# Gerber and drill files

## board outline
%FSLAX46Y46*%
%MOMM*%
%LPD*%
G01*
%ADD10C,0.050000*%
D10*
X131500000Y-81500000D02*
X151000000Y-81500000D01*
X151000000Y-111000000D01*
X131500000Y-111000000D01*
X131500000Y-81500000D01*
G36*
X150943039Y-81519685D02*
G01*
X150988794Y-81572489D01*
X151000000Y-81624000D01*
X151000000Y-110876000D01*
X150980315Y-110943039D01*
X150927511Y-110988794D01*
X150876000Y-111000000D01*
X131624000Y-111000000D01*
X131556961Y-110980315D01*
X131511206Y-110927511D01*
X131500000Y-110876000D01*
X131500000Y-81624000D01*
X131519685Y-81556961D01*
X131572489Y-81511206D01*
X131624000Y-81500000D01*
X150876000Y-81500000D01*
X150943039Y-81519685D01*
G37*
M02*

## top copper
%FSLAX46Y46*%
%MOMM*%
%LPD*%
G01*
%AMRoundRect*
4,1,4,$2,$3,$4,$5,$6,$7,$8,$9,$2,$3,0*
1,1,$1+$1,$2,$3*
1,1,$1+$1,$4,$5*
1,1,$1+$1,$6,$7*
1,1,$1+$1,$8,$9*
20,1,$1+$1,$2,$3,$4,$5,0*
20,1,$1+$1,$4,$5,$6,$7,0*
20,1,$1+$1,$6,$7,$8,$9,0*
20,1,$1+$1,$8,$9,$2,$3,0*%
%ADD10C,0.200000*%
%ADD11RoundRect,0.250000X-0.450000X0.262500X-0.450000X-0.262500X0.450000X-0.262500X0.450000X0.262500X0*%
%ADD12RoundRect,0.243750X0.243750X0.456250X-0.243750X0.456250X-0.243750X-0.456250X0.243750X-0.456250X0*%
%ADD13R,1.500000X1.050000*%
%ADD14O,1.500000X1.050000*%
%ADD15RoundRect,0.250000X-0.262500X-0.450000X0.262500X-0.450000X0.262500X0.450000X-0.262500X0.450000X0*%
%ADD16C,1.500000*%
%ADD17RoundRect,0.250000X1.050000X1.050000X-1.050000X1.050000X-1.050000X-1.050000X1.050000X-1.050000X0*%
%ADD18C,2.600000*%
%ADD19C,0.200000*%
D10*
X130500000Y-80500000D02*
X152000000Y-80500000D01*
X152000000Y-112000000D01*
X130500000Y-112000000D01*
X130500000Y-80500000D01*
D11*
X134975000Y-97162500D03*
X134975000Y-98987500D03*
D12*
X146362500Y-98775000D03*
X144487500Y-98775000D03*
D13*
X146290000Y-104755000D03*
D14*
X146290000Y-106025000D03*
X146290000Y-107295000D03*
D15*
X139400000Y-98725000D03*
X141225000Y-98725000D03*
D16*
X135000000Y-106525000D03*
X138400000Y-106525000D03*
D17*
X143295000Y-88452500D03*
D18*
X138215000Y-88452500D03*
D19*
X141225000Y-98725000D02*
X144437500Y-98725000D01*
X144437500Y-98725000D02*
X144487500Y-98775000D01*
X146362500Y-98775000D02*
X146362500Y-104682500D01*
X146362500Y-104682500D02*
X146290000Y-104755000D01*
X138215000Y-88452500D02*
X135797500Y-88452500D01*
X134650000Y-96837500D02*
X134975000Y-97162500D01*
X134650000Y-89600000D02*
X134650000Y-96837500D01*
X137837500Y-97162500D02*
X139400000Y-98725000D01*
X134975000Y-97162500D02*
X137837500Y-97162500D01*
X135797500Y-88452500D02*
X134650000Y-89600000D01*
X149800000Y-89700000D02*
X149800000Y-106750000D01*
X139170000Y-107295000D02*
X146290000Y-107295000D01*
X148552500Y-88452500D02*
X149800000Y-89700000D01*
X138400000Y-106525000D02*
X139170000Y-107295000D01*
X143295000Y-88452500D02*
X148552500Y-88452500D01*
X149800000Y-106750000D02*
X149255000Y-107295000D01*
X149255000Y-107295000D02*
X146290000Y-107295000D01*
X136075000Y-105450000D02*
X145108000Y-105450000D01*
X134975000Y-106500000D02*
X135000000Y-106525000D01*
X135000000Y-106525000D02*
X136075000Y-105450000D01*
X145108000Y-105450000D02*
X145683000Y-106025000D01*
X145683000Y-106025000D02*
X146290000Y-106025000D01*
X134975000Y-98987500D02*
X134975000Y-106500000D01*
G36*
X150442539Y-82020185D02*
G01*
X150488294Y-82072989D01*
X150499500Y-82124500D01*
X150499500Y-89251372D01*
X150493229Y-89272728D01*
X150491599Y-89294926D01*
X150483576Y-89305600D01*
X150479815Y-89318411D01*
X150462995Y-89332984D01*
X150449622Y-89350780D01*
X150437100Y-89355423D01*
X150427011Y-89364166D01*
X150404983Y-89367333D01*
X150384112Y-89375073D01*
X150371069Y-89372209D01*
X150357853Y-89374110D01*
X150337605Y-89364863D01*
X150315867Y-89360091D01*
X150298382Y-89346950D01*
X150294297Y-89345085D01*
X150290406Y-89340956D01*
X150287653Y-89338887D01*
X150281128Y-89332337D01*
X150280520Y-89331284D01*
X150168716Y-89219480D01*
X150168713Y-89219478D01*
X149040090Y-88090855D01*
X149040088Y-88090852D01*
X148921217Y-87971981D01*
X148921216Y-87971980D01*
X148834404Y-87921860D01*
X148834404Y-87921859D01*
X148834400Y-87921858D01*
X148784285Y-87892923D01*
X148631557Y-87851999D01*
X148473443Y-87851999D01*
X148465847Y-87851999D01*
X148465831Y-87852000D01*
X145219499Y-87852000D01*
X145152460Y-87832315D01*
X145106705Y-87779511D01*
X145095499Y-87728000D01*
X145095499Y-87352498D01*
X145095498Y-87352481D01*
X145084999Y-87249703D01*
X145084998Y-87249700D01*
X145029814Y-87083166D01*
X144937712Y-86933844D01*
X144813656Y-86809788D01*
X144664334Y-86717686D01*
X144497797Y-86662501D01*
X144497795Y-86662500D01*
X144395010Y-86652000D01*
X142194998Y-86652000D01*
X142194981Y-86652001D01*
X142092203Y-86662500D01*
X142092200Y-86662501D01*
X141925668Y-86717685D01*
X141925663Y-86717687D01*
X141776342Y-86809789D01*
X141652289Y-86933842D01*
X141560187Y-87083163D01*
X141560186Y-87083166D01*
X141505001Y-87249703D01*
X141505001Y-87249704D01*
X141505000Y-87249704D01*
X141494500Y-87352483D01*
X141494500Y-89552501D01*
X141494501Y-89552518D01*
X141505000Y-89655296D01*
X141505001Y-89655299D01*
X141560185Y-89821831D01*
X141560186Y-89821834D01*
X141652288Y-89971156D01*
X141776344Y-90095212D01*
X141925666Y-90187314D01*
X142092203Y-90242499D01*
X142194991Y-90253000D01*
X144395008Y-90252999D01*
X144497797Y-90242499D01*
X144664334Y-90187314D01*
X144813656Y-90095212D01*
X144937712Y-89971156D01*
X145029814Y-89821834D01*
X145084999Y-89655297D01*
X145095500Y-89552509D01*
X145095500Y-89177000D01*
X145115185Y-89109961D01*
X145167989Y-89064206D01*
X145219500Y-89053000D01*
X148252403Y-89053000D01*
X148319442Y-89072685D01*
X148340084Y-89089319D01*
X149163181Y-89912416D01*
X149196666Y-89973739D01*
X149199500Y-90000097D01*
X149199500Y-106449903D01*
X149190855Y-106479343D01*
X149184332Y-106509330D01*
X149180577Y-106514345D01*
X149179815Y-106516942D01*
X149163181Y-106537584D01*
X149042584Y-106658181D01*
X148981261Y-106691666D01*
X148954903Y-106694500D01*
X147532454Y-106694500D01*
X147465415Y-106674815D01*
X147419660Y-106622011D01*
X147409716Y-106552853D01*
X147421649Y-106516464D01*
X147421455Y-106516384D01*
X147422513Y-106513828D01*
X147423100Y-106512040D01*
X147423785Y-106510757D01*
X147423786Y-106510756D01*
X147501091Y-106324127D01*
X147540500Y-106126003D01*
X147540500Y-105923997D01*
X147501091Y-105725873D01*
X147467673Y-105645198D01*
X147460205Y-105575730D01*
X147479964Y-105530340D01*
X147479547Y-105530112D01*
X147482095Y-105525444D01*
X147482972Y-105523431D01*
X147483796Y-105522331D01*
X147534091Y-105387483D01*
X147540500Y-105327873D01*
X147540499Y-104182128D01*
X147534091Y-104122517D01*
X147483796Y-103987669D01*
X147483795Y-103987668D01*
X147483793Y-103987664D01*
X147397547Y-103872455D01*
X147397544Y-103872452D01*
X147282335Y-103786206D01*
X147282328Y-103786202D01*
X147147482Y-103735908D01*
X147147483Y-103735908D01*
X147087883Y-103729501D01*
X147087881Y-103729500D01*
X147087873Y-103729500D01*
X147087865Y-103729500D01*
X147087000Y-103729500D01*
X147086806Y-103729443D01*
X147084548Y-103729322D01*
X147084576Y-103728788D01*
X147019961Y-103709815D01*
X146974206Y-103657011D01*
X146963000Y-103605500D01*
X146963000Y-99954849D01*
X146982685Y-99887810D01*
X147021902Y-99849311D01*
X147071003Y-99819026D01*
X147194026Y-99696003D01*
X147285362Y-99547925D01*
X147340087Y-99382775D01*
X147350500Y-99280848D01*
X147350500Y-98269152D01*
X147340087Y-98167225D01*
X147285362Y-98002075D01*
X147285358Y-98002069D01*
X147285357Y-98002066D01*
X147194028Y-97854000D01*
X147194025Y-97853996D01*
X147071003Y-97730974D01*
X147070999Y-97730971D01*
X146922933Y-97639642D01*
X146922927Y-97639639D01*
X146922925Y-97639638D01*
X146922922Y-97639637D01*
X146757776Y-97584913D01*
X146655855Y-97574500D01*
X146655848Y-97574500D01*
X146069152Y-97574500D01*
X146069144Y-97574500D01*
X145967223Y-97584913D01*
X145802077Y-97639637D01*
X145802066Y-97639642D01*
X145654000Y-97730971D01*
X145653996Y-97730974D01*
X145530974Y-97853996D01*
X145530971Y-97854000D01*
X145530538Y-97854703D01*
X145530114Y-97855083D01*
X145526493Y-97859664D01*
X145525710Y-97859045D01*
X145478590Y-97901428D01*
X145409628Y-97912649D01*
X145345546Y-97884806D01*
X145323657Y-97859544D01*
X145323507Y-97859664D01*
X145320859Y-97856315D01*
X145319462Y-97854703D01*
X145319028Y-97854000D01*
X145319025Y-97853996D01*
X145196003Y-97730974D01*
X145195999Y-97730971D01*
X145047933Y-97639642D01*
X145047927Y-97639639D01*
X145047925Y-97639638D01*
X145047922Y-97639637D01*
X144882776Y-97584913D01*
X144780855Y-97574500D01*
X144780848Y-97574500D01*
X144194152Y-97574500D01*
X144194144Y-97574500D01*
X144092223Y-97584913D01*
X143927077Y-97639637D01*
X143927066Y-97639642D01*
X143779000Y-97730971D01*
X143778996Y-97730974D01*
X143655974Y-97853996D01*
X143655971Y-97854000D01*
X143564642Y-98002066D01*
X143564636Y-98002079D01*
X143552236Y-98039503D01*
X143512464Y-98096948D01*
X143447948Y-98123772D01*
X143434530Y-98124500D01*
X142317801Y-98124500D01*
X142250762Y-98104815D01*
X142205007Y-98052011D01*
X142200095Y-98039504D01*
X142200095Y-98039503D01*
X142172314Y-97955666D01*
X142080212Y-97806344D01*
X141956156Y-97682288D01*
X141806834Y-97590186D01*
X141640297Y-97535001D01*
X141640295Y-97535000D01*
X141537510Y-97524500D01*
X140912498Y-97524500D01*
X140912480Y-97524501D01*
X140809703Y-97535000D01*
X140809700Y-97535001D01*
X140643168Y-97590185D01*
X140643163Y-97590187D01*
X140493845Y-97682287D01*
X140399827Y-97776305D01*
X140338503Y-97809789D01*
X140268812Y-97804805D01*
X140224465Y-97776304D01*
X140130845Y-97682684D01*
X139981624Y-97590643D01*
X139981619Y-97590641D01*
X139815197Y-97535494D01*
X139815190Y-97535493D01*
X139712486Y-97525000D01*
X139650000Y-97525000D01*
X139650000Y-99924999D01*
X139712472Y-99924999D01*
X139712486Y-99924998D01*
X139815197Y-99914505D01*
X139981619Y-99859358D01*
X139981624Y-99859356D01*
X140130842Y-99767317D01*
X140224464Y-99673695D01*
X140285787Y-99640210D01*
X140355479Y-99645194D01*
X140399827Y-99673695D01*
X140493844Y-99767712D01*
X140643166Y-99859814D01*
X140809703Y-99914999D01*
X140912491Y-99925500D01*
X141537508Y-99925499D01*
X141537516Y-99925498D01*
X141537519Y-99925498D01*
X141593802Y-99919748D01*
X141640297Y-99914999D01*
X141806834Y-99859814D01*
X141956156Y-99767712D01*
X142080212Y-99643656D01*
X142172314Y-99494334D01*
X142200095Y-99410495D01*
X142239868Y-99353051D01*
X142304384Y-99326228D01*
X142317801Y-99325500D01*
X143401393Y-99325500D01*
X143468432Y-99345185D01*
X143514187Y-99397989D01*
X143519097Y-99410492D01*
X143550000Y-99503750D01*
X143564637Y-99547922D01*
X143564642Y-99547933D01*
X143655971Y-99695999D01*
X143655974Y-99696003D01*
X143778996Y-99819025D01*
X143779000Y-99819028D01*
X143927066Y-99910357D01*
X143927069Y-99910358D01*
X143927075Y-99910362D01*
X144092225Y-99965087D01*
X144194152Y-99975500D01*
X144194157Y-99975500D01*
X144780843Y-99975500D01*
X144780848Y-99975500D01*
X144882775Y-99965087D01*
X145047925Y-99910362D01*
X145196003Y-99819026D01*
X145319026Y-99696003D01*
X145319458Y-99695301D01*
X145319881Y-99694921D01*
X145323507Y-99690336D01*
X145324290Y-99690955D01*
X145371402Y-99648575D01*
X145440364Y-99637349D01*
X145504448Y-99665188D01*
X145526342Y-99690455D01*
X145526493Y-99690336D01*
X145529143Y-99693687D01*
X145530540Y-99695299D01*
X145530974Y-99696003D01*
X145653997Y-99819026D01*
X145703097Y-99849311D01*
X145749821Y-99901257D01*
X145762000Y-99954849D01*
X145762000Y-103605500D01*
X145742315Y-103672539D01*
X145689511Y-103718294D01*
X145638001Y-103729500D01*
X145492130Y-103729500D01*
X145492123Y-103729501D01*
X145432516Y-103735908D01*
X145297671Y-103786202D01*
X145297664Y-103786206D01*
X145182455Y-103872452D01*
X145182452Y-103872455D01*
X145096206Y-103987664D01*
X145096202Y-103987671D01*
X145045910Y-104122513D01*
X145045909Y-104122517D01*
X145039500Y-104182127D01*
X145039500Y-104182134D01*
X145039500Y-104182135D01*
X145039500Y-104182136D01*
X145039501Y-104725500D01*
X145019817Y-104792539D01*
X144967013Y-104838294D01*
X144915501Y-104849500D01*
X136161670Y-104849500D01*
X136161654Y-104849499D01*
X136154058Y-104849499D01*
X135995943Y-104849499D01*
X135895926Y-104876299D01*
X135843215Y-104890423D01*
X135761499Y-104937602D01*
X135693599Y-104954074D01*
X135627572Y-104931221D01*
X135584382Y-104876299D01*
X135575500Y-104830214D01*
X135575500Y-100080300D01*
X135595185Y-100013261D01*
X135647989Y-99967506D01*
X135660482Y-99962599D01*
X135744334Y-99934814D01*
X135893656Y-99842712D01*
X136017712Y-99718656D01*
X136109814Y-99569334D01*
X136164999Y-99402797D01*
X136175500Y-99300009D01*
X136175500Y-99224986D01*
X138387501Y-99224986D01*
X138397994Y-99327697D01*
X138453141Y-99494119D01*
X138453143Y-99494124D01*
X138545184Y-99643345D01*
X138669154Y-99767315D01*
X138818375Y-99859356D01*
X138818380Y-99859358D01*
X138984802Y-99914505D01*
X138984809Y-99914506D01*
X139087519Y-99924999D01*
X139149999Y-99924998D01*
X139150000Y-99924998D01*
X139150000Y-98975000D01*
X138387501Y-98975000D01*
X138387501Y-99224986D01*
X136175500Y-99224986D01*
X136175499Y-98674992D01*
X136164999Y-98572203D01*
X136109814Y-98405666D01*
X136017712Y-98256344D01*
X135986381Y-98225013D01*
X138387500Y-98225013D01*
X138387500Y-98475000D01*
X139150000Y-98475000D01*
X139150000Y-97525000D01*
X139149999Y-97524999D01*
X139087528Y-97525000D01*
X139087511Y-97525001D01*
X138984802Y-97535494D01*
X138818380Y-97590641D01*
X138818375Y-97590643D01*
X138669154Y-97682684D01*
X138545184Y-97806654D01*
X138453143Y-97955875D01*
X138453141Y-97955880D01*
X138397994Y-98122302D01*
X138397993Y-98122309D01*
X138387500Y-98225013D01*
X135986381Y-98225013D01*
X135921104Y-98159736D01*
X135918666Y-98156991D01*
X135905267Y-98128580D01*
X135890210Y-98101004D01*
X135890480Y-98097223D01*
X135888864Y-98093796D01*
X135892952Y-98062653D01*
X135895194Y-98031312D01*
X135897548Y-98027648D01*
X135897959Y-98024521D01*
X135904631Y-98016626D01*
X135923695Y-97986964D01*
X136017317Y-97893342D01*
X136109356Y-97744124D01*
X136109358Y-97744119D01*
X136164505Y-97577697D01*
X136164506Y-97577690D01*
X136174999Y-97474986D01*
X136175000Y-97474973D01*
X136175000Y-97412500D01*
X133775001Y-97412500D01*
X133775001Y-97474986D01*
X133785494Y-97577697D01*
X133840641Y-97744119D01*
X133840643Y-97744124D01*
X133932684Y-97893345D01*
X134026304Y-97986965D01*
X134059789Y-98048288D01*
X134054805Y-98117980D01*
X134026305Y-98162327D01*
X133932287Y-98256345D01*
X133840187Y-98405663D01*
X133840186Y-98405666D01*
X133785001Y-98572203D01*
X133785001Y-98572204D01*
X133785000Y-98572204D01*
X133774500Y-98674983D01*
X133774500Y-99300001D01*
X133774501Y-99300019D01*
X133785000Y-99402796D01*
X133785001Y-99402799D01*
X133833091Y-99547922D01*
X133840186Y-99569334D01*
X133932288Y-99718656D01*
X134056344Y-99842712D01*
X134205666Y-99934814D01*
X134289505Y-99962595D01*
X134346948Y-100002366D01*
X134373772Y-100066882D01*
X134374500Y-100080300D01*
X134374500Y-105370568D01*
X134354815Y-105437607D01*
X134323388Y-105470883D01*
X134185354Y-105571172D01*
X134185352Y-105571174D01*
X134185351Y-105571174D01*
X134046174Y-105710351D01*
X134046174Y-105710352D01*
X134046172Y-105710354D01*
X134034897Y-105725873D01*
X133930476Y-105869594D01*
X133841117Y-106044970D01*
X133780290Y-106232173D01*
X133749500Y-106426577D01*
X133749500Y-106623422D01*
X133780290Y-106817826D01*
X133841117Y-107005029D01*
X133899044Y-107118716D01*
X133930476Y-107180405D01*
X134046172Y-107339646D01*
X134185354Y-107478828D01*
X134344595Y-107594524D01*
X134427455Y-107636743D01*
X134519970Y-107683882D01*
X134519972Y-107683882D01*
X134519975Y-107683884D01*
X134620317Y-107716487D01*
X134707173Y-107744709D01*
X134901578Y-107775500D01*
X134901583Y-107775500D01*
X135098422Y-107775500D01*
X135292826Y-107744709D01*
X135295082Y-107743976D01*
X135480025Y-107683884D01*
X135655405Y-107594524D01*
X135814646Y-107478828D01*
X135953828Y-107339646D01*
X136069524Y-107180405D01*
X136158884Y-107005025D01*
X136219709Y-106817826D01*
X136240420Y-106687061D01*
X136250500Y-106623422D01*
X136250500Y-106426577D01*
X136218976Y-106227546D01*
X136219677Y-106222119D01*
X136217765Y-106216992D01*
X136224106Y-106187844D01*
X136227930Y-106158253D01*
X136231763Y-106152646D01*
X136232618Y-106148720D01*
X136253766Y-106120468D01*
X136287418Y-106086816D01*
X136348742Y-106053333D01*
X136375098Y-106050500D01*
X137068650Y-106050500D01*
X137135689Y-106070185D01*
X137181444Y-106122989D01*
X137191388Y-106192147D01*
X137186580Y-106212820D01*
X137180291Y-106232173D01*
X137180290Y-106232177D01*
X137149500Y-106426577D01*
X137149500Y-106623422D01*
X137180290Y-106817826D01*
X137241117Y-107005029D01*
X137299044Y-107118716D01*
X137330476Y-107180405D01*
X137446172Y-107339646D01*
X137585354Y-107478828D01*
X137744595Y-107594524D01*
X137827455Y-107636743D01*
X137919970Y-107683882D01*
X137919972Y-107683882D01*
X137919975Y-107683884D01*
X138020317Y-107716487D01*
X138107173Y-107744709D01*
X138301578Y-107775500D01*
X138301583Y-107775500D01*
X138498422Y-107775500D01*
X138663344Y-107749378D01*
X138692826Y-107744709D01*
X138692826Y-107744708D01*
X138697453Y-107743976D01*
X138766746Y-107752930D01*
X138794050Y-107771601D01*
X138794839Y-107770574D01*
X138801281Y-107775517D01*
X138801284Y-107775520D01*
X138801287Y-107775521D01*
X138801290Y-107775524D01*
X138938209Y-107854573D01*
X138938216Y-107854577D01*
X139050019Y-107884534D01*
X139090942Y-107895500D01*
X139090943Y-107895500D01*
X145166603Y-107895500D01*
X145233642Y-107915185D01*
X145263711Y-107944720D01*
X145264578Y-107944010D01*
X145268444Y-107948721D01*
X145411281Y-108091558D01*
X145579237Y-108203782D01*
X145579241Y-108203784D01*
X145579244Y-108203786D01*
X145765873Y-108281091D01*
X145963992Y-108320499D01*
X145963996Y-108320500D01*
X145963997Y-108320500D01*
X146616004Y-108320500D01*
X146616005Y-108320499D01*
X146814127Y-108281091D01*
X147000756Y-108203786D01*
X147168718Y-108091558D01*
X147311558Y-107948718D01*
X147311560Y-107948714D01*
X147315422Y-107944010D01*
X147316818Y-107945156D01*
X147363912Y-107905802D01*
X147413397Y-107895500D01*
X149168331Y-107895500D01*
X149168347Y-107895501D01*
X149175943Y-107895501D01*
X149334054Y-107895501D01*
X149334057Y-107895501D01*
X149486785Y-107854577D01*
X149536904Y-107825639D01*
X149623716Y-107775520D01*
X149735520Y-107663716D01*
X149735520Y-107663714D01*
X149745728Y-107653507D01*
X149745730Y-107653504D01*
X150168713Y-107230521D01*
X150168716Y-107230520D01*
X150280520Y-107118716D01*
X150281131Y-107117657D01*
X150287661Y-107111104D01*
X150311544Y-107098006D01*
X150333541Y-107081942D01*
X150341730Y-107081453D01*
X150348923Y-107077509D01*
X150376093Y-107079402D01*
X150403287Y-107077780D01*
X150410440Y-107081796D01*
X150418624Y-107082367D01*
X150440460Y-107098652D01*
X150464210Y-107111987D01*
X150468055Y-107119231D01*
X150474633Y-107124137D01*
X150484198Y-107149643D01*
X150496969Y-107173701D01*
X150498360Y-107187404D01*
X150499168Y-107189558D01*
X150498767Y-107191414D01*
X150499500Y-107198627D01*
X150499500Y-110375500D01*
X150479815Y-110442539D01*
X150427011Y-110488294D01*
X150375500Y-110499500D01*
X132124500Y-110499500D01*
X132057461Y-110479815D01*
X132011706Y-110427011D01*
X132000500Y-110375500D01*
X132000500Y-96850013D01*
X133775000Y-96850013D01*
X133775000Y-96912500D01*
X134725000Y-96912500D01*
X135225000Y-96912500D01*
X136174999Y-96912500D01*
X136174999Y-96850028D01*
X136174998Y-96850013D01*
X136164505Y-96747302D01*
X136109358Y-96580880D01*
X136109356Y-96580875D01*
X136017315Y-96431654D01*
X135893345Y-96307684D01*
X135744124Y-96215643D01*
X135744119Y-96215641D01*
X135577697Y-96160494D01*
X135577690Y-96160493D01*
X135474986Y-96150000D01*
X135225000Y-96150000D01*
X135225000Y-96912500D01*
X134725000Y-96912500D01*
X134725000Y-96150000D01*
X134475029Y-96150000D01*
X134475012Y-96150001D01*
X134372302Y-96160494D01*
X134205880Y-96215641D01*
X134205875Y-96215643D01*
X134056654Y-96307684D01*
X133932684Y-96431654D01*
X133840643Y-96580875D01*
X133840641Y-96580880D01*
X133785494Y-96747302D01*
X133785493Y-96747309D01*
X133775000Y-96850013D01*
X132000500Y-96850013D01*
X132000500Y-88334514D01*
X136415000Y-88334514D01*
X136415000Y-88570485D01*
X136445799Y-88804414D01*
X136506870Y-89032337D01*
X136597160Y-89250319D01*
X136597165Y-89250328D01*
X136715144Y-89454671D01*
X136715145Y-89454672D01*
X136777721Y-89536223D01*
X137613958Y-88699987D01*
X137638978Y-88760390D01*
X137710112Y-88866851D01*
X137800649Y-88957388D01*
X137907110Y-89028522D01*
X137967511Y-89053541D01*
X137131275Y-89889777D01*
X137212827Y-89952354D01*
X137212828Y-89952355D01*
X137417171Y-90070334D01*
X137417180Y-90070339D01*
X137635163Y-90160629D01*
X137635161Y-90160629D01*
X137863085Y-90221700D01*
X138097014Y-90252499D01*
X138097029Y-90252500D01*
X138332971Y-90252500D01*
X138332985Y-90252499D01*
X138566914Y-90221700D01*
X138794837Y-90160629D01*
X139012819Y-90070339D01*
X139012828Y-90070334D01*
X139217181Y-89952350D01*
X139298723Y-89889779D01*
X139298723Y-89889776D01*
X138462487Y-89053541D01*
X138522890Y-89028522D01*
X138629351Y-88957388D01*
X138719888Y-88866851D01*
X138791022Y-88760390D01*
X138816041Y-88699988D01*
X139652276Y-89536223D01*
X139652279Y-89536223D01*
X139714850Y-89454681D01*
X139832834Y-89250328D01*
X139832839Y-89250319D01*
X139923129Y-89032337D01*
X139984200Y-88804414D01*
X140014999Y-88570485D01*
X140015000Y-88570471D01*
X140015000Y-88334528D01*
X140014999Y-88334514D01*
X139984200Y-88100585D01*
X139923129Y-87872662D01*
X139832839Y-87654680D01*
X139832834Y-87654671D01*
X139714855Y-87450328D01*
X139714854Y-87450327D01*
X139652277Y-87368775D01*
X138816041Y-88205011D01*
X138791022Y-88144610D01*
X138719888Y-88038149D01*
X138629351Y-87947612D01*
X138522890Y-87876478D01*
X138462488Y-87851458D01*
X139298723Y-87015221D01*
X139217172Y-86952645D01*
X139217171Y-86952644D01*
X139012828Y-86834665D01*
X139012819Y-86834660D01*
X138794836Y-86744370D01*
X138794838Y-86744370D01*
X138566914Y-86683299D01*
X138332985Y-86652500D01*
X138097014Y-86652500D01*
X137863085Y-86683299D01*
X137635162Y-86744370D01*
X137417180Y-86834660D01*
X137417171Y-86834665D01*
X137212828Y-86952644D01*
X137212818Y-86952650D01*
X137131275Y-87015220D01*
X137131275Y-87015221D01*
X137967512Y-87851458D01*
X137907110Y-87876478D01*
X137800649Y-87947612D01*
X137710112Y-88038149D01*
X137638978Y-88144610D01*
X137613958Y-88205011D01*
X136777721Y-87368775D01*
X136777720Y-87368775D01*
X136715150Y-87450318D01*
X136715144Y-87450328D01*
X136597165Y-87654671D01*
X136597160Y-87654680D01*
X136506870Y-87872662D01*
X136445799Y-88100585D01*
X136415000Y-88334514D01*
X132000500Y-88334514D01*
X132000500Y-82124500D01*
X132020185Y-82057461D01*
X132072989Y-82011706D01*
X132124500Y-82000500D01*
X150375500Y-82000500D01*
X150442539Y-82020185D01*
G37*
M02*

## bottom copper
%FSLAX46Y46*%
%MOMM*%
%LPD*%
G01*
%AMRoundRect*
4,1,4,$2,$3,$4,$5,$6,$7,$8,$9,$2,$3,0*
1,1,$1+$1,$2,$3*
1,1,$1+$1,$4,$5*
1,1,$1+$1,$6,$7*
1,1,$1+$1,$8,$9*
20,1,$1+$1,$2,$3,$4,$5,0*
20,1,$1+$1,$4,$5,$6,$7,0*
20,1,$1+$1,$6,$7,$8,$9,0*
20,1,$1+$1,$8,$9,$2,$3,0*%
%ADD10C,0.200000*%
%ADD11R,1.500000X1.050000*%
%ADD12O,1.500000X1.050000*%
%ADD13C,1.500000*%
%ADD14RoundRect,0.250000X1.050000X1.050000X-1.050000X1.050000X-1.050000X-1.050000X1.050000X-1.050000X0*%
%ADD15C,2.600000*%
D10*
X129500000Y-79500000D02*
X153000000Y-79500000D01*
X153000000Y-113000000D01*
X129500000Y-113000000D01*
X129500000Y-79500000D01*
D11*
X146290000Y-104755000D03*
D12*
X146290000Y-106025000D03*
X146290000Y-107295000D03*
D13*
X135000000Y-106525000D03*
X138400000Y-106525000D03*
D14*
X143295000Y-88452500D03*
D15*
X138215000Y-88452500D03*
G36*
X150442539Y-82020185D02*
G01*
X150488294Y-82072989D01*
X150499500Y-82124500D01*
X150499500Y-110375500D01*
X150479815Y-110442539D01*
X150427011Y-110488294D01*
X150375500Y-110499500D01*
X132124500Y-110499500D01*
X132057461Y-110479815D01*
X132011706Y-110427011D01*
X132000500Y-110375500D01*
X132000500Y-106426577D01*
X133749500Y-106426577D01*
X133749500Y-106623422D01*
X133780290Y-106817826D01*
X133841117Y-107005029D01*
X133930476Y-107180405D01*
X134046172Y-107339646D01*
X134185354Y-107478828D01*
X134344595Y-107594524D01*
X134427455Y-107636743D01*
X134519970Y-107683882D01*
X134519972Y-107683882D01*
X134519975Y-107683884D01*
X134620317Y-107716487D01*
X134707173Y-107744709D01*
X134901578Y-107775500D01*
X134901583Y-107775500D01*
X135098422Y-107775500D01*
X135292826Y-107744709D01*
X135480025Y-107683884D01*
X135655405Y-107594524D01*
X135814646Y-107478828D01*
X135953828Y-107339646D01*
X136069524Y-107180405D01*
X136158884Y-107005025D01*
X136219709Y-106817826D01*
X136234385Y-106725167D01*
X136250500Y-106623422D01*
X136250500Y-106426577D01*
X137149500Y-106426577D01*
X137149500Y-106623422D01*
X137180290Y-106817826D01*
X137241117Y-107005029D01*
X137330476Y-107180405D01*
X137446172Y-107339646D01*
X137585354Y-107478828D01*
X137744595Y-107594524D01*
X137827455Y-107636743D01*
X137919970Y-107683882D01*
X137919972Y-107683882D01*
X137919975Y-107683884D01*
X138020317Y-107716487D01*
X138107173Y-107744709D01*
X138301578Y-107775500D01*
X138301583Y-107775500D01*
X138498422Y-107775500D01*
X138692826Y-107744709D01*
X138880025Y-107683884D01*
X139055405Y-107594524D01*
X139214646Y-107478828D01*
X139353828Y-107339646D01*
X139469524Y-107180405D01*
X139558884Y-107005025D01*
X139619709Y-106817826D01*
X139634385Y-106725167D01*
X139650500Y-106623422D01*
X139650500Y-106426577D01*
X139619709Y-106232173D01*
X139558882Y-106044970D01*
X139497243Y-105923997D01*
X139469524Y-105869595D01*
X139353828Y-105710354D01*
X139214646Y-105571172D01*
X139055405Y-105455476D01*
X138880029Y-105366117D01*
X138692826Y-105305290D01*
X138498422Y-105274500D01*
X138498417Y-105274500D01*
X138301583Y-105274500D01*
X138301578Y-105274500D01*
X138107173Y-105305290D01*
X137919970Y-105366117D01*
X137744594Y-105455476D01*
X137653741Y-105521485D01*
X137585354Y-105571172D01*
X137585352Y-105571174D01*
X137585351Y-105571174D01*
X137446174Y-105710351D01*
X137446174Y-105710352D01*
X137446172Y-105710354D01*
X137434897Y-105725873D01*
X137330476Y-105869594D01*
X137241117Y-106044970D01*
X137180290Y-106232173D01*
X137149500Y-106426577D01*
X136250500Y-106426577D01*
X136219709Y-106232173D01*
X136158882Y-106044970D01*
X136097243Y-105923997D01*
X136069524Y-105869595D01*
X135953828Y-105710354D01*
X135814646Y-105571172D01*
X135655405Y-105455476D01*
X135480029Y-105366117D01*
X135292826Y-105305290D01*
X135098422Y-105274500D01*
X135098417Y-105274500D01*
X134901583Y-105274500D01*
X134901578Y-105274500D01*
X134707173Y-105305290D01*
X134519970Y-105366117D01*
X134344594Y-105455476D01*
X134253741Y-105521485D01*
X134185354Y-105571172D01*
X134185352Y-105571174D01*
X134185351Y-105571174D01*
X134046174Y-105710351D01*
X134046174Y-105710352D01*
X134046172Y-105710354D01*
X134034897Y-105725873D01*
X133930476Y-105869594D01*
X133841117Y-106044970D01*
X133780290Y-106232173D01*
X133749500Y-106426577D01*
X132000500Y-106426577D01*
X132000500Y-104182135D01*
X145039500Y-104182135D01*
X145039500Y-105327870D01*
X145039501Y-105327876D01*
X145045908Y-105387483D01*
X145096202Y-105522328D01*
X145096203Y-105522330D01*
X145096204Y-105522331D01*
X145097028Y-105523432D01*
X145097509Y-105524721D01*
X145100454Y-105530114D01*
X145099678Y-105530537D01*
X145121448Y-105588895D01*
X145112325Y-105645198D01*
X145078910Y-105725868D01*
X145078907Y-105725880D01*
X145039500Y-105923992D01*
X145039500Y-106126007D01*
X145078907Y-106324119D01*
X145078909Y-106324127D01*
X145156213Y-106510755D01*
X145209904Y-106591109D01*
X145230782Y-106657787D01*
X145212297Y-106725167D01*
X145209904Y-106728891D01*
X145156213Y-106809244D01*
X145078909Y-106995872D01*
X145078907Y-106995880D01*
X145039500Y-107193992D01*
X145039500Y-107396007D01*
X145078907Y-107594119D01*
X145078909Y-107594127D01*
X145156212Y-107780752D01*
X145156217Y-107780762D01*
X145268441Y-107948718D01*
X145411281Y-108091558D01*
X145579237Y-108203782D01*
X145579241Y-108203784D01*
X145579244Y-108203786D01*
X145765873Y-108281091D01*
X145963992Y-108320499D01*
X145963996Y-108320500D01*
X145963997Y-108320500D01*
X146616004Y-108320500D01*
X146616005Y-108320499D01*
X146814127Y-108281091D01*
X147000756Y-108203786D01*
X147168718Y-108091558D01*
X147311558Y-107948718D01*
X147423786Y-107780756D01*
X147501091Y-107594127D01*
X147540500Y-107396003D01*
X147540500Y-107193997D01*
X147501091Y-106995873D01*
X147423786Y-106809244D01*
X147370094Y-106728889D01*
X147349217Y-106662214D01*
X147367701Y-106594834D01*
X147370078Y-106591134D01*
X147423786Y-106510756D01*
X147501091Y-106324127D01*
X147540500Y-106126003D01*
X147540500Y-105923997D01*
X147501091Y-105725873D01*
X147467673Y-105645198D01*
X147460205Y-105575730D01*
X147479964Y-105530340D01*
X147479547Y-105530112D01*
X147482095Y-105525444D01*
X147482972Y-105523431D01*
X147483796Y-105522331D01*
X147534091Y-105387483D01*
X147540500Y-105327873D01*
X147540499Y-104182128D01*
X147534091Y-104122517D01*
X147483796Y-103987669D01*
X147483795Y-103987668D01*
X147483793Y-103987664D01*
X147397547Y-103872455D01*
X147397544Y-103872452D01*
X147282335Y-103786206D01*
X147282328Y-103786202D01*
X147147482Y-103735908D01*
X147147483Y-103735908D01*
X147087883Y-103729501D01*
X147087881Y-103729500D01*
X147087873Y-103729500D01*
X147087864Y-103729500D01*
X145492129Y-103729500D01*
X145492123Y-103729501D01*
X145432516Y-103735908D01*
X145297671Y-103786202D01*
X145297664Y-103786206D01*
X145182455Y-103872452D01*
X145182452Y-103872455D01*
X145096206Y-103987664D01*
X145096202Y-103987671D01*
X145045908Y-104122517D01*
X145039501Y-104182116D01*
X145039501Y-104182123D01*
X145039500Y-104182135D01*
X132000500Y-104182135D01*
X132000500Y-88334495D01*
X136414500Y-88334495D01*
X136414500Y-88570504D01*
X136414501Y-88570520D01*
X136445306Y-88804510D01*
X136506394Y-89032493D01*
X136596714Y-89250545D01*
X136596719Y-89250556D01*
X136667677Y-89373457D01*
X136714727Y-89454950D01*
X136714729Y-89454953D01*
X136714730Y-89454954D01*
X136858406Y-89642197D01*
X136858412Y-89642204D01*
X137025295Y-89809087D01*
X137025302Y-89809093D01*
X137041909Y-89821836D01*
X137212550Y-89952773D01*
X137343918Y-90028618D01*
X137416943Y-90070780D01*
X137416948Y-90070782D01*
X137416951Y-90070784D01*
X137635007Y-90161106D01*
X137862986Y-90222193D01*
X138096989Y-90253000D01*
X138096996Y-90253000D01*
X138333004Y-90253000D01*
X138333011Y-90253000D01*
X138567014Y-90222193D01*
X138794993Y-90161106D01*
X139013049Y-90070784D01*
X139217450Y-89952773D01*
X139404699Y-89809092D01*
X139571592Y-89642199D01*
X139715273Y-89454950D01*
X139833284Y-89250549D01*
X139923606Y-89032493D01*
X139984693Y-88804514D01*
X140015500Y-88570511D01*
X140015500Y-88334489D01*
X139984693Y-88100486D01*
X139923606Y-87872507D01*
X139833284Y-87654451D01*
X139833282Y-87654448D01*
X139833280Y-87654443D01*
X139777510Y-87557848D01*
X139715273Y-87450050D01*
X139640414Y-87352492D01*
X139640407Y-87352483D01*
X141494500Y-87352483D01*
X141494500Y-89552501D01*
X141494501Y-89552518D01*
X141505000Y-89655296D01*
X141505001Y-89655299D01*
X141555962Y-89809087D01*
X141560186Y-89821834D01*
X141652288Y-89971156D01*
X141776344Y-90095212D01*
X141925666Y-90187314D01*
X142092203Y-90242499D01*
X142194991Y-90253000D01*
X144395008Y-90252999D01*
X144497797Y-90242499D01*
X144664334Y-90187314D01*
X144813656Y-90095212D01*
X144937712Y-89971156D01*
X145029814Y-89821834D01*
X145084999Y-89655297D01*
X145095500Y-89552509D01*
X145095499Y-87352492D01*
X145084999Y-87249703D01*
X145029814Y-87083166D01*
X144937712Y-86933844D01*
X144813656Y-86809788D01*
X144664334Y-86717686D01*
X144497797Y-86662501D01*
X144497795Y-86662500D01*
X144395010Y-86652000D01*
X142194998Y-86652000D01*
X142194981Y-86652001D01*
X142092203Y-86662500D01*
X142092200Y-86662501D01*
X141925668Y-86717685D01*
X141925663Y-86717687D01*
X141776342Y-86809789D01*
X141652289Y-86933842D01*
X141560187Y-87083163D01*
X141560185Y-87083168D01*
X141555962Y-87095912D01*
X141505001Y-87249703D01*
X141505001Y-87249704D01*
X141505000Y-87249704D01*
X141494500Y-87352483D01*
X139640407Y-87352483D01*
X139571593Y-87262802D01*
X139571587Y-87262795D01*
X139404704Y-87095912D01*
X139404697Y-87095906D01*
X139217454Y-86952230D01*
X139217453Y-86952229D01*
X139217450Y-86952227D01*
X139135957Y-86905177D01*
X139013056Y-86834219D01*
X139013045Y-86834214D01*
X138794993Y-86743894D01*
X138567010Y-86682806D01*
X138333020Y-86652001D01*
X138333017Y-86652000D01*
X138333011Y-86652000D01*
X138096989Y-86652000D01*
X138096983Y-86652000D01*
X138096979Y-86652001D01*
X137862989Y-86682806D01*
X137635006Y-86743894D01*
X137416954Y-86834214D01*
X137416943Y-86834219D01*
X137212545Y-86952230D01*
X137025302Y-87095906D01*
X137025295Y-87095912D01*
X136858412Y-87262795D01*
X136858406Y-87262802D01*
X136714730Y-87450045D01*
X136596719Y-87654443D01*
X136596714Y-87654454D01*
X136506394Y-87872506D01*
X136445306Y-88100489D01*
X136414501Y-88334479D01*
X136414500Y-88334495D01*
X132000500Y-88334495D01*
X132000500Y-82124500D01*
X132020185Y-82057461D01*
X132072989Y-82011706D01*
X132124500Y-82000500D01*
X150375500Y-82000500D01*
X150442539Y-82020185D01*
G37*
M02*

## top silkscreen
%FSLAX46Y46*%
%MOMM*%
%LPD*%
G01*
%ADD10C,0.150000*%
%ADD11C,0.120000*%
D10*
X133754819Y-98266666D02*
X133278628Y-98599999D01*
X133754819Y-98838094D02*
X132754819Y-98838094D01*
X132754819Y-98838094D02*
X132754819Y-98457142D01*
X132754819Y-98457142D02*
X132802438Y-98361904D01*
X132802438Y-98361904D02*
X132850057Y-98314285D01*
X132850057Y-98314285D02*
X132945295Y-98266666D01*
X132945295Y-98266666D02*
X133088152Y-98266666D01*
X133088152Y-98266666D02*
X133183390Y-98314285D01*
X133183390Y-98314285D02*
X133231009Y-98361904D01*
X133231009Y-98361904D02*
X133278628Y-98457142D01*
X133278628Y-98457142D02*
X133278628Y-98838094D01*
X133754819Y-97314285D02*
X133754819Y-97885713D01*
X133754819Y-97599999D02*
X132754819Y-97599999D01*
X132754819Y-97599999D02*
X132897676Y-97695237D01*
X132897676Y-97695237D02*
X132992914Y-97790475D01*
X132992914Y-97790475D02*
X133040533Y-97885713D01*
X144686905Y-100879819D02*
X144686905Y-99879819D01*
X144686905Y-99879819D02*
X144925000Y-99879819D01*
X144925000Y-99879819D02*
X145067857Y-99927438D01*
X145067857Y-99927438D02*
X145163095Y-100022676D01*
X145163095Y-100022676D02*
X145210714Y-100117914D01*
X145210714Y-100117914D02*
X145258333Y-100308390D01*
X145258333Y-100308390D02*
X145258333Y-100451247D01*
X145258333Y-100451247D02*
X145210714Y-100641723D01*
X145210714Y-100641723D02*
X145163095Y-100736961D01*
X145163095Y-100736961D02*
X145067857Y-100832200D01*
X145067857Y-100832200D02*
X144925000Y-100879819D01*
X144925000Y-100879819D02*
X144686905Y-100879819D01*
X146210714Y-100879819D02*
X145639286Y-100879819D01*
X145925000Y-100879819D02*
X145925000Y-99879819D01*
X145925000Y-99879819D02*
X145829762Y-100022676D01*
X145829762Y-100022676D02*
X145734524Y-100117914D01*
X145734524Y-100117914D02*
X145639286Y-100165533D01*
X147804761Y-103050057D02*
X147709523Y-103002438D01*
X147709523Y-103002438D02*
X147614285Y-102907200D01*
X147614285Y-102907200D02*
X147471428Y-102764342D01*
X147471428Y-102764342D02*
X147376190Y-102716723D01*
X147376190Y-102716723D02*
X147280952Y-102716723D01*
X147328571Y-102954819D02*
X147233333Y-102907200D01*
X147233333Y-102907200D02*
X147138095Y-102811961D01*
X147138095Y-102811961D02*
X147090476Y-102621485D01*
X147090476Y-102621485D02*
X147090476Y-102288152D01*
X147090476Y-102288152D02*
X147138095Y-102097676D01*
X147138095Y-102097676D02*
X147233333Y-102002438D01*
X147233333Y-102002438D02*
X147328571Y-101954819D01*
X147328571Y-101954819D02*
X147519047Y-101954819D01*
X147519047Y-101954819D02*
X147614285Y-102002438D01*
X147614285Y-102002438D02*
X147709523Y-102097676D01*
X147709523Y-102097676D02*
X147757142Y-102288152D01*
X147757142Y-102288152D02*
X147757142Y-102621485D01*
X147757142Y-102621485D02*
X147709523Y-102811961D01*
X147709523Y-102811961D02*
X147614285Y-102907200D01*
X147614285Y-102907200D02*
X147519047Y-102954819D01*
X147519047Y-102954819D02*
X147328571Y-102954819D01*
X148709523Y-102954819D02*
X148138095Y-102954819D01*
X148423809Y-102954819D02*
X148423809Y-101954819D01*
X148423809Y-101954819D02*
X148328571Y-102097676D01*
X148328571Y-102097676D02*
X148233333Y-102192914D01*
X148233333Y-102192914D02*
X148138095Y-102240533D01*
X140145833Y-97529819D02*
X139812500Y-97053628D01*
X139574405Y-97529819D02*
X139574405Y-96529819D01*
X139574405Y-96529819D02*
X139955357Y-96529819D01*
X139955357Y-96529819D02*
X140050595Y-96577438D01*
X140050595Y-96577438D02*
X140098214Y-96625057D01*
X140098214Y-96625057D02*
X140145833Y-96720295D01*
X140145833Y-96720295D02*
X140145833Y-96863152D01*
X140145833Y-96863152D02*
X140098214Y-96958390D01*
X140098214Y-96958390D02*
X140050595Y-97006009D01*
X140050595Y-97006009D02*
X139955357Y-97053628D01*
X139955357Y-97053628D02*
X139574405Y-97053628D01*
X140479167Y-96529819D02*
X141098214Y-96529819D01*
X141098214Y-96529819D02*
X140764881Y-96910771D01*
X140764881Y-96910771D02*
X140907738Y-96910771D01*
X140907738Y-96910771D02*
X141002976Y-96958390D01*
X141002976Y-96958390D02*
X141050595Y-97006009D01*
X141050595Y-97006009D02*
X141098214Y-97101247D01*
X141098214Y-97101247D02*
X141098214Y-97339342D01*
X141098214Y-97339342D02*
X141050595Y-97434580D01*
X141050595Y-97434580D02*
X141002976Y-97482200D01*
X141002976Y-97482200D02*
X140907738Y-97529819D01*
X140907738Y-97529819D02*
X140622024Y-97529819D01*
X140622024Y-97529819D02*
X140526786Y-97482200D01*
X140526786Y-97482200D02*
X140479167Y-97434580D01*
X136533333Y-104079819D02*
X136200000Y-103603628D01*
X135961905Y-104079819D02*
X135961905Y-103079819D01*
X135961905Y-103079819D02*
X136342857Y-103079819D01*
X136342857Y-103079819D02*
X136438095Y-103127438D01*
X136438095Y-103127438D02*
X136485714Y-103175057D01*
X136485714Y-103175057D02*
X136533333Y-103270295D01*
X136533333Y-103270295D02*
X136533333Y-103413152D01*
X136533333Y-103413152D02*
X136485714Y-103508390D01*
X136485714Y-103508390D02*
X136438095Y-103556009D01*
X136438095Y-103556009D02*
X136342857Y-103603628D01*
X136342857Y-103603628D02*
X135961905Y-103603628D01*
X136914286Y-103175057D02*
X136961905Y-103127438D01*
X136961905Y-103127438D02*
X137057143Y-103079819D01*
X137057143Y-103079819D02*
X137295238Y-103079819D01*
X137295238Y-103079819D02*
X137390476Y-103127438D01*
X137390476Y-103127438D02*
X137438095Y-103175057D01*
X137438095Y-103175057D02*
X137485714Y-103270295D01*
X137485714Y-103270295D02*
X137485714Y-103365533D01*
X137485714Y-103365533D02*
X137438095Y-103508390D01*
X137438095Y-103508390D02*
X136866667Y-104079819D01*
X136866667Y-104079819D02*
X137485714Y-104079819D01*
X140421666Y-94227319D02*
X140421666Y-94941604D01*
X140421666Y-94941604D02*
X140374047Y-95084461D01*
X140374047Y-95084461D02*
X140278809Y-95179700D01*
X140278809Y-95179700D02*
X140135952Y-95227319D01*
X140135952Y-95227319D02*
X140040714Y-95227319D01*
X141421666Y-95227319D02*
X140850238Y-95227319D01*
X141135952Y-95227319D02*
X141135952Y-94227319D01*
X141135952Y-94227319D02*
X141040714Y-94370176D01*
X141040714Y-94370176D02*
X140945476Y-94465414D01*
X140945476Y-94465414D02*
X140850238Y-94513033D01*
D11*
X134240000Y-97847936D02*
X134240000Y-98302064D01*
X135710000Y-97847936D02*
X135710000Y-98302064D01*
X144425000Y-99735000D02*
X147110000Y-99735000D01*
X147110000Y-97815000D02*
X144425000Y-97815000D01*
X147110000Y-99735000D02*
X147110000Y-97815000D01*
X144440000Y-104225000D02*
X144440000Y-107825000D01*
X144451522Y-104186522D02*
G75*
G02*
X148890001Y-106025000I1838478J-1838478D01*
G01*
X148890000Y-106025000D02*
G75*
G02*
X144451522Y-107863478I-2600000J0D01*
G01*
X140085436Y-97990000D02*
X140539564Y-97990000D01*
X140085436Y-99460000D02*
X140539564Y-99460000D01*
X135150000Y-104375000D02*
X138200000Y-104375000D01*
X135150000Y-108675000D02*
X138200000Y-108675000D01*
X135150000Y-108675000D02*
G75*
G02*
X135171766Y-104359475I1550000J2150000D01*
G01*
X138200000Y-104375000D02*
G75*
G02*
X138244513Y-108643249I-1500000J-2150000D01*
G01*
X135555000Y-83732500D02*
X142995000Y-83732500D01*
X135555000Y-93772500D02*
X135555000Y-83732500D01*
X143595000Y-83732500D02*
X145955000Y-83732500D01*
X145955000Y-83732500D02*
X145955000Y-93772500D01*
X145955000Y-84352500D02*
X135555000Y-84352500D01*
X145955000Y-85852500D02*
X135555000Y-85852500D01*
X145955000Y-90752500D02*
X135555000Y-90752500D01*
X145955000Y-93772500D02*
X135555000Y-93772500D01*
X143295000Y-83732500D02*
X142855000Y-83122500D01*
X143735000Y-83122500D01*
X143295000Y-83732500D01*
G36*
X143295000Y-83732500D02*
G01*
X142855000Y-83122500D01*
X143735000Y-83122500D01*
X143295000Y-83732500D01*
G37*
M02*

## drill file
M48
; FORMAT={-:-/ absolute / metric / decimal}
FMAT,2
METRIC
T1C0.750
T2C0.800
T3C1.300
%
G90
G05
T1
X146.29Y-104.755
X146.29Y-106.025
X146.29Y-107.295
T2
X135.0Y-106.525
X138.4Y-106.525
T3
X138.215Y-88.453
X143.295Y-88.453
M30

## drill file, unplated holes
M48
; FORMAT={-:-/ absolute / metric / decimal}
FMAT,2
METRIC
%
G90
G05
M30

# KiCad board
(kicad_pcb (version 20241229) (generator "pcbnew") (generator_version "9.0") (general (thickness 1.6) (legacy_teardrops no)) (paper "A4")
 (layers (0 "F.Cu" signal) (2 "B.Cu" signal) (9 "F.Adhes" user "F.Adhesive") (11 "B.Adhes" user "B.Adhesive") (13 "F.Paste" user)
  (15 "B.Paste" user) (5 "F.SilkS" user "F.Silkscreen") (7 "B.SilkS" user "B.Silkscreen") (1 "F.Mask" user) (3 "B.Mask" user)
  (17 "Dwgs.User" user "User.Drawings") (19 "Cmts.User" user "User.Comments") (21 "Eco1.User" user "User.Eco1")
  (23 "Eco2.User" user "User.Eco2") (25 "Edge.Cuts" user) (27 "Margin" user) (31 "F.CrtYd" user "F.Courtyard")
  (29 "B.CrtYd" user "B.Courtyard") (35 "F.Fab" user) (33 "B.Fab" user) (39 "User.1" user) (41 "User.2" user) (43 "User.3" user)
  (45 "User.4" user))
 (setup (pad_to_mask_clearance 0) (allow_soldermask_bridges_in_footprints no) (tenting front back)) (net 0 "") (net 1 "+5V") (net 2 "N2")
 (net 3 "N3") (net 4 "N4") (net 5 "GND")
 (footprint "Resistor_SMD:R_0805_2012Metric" (layer "F.Cu") (at 134.975 98.075 -90)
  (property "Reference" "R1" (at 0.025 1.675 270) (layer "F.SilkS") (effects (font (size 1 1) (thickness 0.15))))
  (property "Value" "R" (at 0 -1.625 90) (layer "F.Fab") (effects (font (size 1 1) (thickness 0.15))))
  (fp_line (start -0.227064 0.735) (end 0.227064 0.735) (stroke (width 0.12) (type solid)) (layer "F.SilkS"))
  (fp_line (start -0.227064 -0.735) (end 0.227064 -0.735) (stroke (width 0.12) (type solid)) (layer "F.SilkS"))
  (pad "1" smd roundrect (at -0.9125 0 270) (size 1.025 1.4) (layers "F.Cu" "F.Mask" "F.Paste") (roundrect_rratio 0.243902) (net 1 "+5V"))
  (pad "2" smd roundrect (at 0.9125 0 270) (size 1.025 1.4) (layers "F.Cu" "F.Mask" "F.Paste") (roundrect_rratio 0.243902) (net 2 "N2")))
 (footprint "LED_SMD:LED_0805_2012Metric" (layer "F.Cu") (at 145.425 98.775 180)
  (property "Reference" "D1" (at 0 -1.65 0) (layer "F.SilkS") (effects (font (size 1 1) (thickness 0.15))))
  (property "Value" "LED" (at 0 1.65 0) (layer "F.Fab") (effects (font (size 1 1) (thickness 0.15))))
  (fp_line (start 1 -0.96) (end -1.685 -0.96) (stroke (width 0.12) (type solid)) (layer "F.SilkS"))
  (fp_line (start -1.685 0.96) (end 1 0.96) (stroke (width 0.12) (type solid)) (layer "F.SilkS"))
  (fp_line (start -1.685 -0.96) (end -1.685 0.96) (stroke (width 0.12) (type solid)) (layer "F.SilkS"))
  (pad "1" smd roundrect (at -0.9375 0 180) (size 0.975 1.4) (layers "F.Cu" "F.Mask" "F.Paste") (roundrect_rratio 0.25) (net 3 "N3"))
  (pad "2" smd roundrect (at 0.9375 0 180) (size 0.975 1.4) (layers "F.Cu" "F.Mask" "F.Paste") (roundrect_rratio 0.25) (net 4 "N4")))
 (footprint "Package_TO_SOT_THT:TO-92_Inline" (layer "F.Cu") (at 146.29 104.755 -90)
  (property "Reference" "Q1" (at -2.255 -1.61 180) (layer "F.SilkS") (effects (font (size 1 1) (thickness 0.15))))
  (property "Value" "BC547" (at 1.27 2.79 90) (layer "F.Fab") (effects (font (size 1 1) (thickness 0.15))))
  (fp_line (start -0.53 1.85) (end 3.07 1.85) (stroke (width 0.12) (type solid)) (layer "F.SilkS"))
  (fp_arc (start -0.568478 1.838478) (mid -1.132087 -0.994977) (end 1.27 -2.6) (stroke (width 0.12) (type solid)) (layer "F.SilkS"))
  (fp_arc (start 1.27 -2.6) (mid 3.672087 -0.994977) (end 3.108478 1.838478) (stroke (width 0.12) (type solid)) (layer "F.SilkS"))
  (pad "1" thru_hole rect (at 0 0 270) (size 1.05 1.5) (drill 0.75) (layers "*.Cu" "*.Mask") (remove_unused_layers no) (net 3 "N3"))
  (pad "2" thru_hole oval (at 1.27 0 270) (size 1.05 1.5) (drill 0.75) (layers "*.Cu" "*.Mask") (remove_unused_layers no) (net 2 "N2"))
  (pad "3" thru_hole oval (at 2.54 0 270) (size 1.05 1.5) (drill 0.75) (layers "*.Cu" "*.Mask") (remove_unused_layers no) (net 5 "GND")))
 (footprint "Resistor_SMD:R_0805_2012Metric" (layer "F.Cu") (at 140.3125 98.725)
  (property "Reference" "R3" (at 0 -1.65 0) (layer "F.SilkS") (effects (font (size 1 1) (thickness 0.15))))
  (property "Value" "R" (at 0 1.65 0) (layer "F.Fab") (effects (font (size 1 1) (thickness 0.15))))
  (fp_line (start -0.227064 -0.735) (end 0.227064 -0.735) (stroke (width 0.12) (type solid)) (layer "F.SilkS"))
  (fp_line (start -0.227064 0.735) (end 0.227064 0.735) (stroke (width 0.12) (type solid)) (layer "F.SilkS"))
  (pad "1" smd roundrect (at -0.9125 0) (size 1.025 1.4) (layers "F.Cu" "F.Mask" "F.Paste") (roundrect_rratio 0.243902) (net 1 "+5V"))
  (pad "2" smd roundrect (at 0.9125 0) (size 1.025 1.4) (layers "F.Cu" "F.Mask" "F.Paste") (roundrect_rratio 0.243902) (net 4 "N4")))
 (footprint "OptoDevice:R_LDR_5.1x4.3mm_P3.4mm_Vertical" (layer "F.Cu") (at 135 106.525)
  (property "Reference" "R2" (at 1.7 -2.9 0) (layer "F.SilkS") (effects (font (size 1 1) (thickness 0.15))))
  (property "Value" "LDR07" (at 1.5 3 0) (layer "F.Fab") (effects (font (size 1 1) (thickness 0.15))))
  (fp_line (start 0.15 -2.15) (end 3.2 -2.15) (stroke (width 0.12) (type solid)) (layer "F.SilkS"))
  (fp_line (start 0.15 2.15) (end 3.2 2.15) (stroke (width 0.12) (type solid)) (layer "F.SilkS"))
  (fp_arc (start 0.15 2.15) (mid -0.950438 -0.013368) (end 0.171766 -2.165525) (stroke (width 0.12) (type solid)) (layer "F.SilkS"))
  (fp_arc (start 3.2 -2.15) (mid 4.321403 -0.027338) (end 3.244513 2.118249) (stroke (width 0.12) (type solid)) (layer "F.SilkS"))
  (pad "1" thru_hole circle (at 0 0) (size 1.5 1.5) (drill 0.8) (layers "*.Cu" "*.Mask") (remove_unused_layers no) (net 2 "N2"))
  (pad "2" thru_hole circle (at 3.4 0) (size 1.5 1.5) (drill 0.8) (layers "*.Cu" "*.Mask") (remove_unused_layers no) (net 5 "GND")))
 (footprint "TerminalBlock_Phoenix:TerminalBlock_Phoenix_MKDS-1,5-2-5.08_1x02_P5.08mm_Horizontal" (layer "F.Cu") (at 143.295 88.4525 180)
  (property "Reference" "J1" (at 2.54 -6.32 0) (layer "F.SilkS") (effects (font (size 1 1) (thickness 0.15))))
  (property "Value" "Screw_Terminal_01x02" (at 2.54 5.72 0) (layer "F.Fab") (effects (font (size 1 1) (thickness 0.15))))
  (fp_line (start 7.74 4.72) (end 0.3 4.72) (stroke (width 0.12) (type solid)) (layer "F.SilkS"))
  (fp_line (start 7.74 -5.32) (end 7.74 4.72) (stroke (width 0.12) (type solid)) (layer "F.SilkS"))
  (fp_line (start -0.3 4.72) (end -2.66 4.72) (stroke (width 0.12) (type solid)) (layer "F.SilkS"))
  (fp_line (start -2.66 4.72) (end -2.66 -5.32) (stroke (width 0.12) (type solid)) (layer "F.SilkS"))
  (fp_line (start -2.66 4.1) (end 7.74 4.1) (stroke (width 0.12) (type solid)) (layer "F.SilkS"))
  (fp_line (start -2.66 2.6) (end 7.74 2.6) (stroke (width 0.12) (type solid)) (layer "F.SilkS"))
  (fp_line (start -2.66 -2.3) (end 7.74 -2.3) (stroke (width 0.12) (type solid)) (layer "F.SilkS"))
  (fp_line (start -2.66 -5.32) (end 7.74 -5.32) (stroke (width 0.12) (type solid)) (layer "F.SilkS"))
  (fp_poly (pts (xy 0 4.72) (xy 0.44 5.33) (xy -0.44 5.33)) (stroke (width 0.12) (type solid)) (fill yes) (layer "F.SilkS"))
  (pad "1" thru_hole roundrect (at 0 0 180) (size 2.6 2.6) (drill 1.3) (layers "*.Cu" "*.Mask") (remove_unused_layers no)
   (roundrect_rratio 0.096154) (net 5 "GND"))
  (pad "2" thru_hole circle (at 5.08 0 180) (size 2.6 2.6) (drill 1.3) (layers "*.Cu" "*.Mask") (remove_unused_layers no) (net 1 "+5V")))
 (gr_rect (start 130.5 80.5) (end 152 112) (stroke (width 0.2) (type default)) (fill no) (layer "F.Cu"))
 (gr_rect (start 129.5 79.5) (end 153 113) (stroke (width 0.2) (type default)) (fill no) (layer "B.Cu"))
 (gr_rect (start 131.5 81.5) (end 151 111) (stroke (width 0.05) (type default)) (fill no) (layer "Edge.Cuts"))
 (segment (start 141.225 98.725) (end 144.4375 98.725) (width 0.2) (layer "F.Cu") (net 4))
 (segment (start 144.4375 98.725) (end 144.4875 98.775) (width 0.2) (layer "F.Cu") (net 4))
 (segment (start 146.3625 98.775) (end 146.3625 104.6825) (width 0.2) (layer "F.Cu") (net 3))
 (segment (start 146.3625 104.6825) (end 146.29 104.755) (width 0.2) (layer "F.Cu") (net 3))
 (segment (start 138.215 88.4525) (end 135.7975 88.4525) (width 0.2) (layer "F.Cu") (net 1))
 (segment (start 134.65 96.8375) (end 134.975 97.1625) (width 0.2) (layer "F.Cu") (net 1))
 (segment (start 134.65 89.6) (end 134.65 96.8375) (width 0.2) (layer "F.Cu") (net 1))
 (segment (start 137.8375 97.1625) (end 139.4 98.725) (width 0.2) (layer "F.Cu") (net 1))
 (segment (start 134.975 97.1625) (end 137.8375 97.1625) (width 0.2) (layer "F.Cu") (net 1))
 (segment (start 135.7975 88.4525) (end 134.65 89.6) (width 0.2) (layer "F.Cu") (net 1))
 (segment (start 149.8 89.7) (end 149.8 106.75) (width 0.2) (layer "F.Cu") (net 5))
 (segment (start 139.17 107.295) (end 146.29 107.295) (width 0.2) (layer "F.Cu") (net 5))
 (segment (start 148.5525 88.4525) (end 149.8 89.7) (width 0.2) (layer "F.Cu") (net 5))
 (segment (start 138.4 106.525) (end 139.17 107.295) (width 0.2) (layer "F.Cu") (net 5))
 (segment (start 143.295 88.4525) (end 148.5525 88.4525) (width 0.2) (layer "F.Cu") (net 5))
 (segment (start 149.8 106.75) (end 149.255 107.295) (width 0.2) (layer "F.Cu") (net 5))
 (segment (start 149.255 107.295) (end 146.29 107.295) (width 0.2) (layer "F.Cu") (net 5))
 (segment (start 136.075 105.45) (end 145.108 105.45) (width 0.2) (layer "F.Cu") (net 2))
 (segment (start 134.975 106.5) (end 135 106.525) (width 0.2) (layer "F.Cu") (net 2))
 (segment (start 135 106.525) (end 136.075 105.45) (width 0.2) (layer "F.Cu") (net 2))
 (segment (start 145.108 105.45) (end 145.683 106.025) (width 0.2) (layer "F.Cu") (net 2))
 (segment (start 145.683 106.025) (end 146.29 106.025) (width 0.2) (layer "F.Cu") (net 2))
 (segment (start 134.975 98.9875) (end 134.975 106.5) (width 0.2) (layer "F.Cu") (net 2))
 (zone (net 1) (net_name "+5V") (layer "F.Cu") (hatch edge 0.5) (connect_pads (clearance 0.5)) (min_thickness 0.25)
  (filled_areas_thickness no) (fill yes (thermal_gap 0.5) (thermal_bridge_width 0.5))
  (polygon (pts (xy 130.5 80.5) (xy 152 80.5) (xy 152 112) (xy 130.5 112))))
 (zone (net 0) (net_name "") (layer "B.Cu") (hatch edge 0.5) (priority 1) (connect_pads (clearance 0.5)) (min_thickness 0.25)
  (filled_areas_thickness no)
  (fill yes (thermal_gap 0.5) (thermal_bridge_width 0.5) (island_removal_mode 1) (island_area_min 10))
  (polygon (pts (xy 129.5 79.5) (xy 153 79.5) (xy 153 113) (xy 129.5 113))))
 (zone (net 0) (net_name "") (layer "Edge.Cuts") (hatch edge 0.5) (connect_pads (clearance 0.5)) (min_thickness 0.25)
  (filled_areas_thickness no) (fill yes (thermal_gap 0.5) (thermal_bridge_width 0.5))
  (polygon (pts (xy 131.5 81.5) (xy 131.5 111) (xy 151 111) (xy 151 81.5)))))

